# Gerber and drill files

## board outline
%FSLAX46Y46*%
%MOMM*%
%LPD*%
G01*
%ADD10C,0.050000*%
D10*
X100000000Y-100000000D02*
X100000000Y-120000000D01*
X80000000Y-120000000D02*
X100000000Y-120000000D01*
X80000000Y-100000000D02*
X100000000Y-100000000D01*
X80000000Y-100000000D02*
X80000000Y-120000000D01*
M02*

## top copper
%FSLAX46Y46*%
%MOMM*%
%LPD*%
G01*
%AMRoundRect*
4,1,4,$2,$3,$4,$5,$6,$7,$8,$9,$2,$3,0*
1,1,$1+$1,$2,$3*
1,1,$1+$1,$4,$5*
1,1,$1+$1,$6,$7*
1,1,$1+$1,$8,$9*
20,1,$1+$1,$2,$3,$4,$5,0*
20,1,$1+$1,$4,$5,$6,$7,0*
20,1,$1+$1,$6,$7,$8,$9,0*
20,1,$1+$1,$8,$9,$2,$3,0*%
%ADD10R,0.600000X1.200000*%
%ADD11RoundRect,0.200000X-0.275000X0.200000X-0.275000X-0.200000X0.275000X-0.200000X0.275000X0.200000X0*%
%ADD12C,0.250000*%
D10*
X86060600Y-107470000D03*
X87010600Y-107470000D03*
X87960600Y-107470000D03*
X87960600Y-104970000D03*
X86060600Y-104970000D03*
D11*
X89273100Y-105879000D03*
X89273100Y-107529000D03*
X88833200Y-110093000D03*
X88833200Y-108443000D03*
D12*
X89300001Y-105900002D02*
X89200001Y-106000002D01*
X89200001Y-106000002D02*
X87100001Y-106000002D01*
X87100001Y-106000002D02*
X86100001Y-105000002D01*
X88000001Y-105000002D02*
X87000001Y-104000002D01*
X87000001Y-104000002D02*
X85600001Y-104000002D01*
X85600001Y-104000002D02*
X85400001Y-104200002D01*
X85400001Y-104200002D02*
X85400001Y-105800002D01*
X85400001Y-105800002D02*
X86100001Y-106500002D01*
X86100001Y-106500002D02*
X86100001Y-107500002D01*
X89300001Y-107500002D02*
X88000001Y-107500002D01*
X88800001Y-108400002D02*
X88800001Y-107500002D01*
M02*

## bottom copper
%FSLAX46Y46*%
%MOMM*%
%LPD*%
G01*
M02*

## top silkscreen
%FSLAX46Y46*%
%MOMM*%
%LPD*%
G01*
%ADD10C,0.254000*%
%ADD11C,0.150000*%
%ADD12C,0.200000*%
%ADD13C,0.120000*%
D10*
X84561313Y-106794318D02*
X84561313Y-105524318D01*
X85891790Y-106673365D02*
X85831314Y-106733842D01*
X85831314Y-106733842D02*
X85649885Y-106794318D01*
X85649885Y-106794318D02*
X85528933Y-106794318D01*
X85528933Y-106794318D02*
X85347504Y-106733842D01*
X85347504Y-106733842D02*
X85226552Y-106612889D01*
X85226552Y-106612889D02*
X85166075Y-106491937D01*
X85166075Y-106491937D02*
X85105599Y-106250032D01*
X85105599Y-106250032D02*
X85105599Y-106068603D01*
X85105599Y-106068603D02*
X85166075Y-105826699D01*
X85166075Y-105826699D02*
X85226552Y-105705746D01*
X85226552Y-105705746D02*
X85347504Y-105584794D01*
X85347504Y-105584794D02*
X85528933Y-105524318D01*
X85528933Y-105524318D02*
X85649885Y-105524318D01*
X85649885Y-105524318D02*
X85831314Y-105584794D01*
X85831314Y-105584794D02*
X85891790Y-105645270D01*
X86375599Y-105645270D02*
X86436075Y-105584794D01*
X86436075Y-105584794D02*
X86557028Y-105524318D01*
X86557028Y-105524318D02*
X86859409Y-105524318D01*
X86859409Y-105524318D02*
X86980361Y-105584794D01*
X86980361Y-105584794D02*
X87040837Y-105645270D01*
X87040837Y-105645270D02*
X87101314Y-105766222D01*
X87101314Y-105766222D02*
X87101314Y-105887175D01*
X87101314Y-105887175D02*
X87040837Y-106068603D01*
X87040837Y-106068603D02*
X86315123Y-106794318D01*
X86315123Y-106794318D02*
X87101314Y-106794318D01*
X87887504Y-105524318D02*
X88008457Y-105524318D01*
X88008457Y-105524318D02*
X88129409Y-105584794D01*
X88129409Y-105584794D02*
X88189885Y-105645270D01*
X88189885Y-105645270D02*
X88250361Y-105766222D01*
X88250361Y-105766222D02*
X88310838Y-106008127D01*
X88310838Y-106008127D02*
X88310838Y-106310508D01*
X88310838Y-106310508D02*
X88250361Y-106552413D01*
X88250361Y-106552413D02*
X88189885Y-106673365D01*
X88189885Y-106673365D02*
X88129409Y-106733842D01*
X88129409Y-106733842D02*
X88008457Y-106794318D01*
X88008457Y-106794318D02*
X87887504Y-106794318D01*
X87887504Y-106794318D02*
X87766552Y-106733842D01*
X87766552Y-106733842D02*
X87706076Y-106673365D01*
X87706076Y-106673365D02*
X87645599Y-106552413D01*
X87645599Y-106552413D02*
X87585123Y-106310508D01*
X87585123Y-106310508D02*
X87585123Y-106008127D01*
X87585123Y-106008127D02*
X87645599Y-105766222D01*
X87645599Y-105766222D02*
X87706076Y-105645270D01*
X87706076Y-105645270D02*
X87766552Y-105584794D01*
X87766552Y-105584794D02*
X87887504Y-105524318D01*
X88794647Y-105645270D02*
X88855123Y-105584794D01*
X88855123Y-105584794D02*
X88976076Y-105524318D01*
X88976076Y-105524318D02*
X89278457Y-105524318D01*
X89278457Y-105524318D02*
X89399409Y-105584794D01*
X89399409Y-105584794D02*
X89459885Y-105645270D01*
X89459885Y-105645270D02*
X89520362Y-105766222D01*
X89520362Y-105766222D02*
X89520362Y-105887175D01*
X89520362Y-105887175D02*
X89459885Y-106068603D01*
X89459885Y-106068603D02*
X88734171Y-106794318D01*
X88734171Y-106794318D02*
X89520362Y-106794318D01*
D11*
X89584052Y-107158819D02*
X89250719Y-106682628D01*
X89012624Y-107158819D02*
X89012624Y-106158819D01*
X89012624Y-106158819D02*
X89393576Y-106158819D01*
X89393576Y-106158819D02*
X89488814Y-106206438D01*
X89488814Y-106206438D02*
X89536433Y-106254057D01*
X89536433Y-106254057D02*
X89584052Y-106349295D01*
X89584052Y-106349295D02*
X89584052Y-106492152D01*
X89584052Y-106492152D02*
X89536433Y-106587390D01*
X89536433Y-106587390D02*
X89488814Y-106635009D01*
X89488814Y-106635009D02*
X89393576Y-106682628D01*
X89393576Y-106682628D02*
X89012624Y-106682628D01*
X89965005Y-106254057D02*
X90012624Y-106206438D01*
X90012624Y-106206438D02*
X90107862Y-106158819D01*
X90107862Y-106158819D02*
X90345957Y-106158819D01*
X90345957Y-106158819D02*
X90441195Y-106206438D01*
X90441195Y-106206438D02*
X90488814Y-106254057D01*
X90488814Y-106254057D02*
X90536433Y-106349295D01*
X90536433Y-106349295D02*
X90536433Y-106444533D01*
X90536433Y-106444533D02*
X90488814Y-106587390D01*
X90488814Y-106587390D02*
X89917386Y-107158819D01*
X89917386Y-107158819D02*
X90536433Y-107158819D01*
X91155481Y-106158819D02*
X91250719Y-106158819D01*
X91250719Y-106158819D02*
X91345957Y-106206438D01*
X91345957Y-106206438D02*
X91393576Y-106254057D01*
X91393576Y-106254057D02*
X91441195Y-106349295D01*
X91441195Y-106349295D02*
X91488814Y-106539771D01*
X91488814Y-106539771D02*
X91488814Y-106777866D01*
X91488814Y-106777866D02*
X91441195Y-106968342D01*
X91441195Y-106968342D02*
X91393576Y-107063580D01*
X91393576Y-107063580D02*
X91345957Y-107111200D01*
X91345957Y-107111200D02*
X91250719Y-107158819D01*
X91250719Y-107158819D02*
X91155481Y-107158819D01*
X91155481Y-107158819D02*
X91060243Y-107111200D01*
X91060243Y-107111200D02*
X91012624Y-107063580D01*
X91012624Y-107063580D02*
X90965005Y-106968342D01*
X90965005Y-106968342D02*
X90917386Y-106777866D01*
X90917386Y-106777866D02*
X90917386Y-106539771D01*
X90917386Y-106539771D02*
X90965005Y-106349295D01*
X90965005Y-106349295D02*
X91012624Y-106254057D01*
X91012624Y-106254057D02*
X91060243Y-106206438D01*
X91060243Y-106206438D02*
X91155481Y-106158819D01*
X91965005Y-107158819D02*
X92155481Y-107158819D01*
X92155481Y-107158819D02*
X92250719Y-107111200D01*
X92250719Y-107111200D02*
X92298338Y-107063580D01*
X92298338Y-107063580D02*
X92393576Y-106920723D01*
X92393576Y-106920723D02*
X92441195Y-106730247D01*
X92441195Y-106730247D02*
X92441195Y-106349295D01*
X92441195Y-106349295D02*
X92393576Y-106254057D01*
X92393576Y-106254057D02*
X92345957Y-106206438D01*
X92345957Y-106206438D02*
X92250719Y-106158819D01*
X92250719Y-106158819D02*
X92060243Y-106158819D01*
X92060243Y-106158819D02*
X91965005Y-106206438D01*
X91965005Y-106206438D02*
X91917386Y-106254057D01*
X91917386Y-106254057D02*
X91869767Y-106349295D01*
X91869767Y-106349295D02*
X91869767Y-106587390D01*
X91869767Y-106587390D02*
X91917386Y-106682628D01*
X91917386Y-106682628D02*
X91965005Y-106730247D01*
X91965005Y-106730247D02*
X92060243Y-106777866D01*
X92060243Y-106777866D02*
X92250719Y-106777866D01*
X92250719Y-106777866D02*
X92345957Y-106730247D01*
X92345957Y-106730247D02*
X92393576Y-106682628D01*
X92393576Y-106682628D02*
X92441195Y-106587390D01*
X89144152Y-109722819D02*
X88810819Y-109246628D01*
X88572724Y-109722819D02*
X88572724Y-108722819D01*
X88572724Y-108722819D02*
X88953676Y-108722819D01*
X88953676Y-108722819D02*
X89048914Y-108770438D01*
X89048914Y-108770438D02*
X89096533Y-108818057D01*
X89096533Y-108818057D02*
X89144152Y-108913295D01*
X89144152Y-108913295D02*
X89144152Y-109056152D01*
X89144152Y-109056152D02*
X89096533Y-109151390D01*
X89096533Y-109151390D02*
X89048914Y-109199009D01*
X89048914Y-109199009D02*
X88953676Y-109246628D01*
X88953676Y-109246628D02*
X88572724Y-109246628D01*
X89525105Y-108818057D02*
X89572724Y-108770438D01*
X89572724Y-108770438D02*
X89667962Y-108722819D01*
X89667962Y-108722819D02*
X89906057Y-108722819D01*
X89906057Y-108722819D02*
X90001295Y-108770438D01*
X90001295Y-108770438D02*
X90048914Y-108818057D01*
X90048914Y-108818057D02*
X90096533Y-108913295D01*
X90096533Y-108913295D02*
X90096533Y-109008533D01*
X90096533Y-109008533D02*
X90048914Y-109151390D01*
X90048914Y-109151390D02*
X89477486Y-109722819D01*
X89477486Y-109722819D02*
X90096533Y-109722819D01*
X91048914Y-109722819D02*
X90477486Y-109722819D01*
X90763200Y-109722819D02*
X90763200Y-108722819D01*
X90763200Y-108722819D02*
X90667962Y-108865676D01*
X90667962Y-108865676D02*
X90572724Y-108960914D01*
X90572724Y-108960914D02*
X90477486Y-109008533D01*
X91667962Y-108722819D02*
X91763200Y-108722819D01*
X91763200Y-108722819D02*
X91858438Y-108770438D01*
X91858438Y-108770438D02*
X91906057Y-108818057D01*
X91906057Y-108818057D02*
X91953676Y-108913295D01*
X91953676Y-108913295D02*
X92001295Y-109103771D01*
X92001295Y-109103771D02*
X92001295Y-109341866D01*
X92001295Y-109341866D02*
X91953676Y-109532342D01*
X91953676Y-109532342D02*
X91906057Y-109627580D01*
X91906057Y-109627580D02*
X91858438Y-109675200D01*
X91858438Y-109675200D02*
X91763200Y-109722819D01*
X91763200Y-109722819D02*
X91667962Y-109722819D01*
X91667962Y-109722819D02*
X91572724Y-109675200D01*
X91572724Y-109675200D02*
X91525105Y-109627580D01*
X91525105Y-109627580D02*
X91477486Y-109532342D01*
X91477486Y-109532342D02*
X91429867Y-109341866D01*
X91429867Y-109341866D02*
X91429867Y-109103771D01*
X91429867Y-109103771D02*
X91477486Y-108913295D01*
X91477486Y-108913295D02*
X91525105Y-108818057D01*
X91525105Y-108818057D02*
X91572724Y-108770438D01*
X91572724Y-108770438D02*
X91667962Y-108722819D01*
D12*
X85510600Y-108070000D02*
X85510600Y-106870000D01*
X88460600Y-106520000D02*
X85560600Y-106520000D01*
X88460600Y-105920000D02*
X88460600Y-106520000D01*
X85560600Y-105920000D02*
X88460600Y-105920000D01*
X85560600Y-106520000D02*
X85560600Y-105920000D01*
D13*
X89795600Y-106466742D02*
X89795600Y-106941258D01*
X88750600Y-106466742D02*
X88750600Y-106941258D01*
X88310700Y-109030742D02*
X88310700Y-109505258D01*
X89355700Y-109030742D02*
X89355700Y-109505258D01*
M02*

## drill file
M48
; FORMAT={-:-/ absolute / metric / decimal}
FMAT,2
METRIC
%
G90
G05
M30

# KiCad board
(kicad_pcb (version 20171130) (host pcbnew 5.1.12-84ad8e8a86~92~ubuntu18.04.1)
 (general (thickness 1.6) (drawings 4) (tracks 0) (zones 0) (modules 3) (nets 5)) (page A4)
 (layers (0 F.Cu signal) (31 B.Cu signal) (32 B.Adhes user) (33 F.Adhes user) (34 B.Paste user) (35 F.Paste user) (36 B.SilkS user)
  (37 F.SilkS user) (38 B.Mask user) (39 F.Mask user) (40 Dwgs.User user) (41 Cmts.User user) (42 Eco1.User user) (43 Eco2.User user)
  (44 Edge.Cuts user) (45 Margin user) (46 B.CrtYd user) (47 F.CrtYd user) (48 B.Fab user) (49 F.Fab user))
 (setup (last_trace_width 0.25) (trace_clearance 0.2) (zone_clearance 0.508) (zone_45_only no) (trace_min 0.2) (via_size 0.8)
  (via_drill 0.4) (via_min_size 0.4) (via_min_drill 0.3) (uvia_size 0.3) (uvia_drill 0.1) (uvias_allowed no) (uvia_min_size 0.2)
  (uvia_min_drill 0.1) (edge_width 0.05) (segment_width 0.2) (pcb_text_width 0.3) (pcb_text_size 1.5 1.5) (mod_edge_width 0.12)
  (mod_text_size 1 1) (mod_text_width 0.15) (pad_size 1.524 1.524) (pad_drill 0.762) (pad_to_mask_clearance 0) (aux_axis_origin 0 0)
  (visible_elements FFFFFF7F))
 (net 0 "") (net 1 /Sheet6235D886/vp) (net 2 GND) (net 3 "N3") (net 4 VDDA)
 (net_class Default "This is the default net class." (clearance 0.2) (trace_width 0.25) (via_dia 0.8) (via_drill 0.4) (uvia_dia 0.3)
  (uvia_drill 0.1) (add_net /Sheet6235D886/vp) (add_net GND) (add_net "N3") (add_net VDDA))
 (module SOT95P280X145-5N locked (layer F.Cu) (at 87.010600 106.220000 90.000000)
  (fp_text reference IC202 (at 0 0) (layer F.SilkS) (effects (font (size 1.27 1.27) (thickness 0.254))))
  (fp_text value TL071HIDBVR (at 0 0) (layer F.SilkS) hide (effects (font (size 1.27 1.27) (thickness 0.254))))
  (fp_line (start -1.85 -1.5) (end -0.65 -1.5) (layer F.SilkS) (width 0.2))
  (fp_line (start -0.3 1.45) (end -0.3 -1.45) (layer F.SilkS) (width 0.2))
  (fp_line (start 0.3 1.45) (end -0.3 1.45) (layer F.SilkS) (width 0.2))
  (fp_line (start 0.3 -1.45) (end 0.3 1.45) (layer F.SilkS) (width 0.2))
  (fp_line (start -0.3 -1.45) (end 0.3 -1.45) (layer F.SilkS) (width 0.2))
  (pad 1 smd rect (at -1.25 -0.95 180.000000) (size 0.6 1.2) (layers F.Cu F.Mask F.Paste) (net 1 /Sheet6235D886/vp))
  (pad 2 smd rect (at -1.25 0 180.000000) (size 0.6 1.2) (layers F.Cu F.Mask F.Paste) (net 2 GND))
  (pad 3 smd rect (at -1.25 0.95 180.000000) (size 0.6 1.2) (layers F.Cu F.Mask F.Paste) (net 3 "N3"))
  (pad 4 smd rect (at 1.25 0.95 180.000000) (size 0.6 1.2) (layers F.Cu F.Mask F.Paste) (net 1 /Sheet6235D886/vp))
  (pad 5 smd rect (at 1.25 -0.95 180.000000) (size 0.6 1.2) (layers F.Cu F.Mask F.Paste) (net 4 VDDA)))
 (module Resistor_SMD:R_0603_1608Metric (layer F.Cu) (at 89.273100 106.704000 270.000000)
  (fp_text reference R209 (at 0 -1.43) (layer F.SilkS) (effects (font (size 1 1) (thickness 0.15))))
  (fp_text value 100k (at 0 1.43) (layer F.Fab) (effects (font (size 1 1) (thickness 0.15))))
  (fp_line (start -0.237258 -0.5225) (end 0.237258 -0.5225) (layer F.SilkS) (width 0.12))
  (fp_line (start -0.237258 0.5225) (end 0.237258 0.5225) (layer F.SilkS) (width 0.12))
  (pad 1 smd roundrect (at -0.825 0 270.000000) (size 0.8 0.95) (layers F.Cu F.Mask F.Paste) (roundrect_rratio 0.25) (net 4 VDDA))
  (pad 2 smd roundrect (at 0.825 0 270.000000) (size 0.8 0.95) (layers F.Cu F.Mask F.Paste) (roundrect_rratio 0.25) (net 3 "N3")))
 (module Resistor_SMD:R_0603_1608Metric (layer F.Cu) (at 88.833200 109.268000 270.000000)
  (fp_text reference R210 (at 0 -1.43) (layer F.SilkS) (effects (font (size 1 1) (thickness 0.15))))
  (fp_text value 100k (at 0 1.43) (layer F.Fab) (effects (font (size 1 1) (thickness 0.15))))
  (fp_line (start -0.237258 0.5225) (end 0.237258 0.5225) (layer F.SilkS) (width 0.12))
  (fp_line (start -0.237258 -0.5225) (end 0.237258 -0.5225) (layer F.SilkS) (width 0.12))
  (pad 2 smd roundrect (at 0.825 0 270.000000) (size 0.8 0.95) (layers F.Cu F.Mask F.Paste) (roundrect_rratio 0.25) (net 2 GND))
  (pad 1 smd roundrect (at -0.825 0 270.000000) (size 0.8 0.95) (layers F.Cu F.Mask F.Paste) (roundrect_rratio 0.25) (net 3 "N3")))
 (gr_line (start 100 100) (end 100 120) (layer Edge.Cuts) (width 0.05))
 (gr_line (start 80 120) (end 100 120) (layer Edge.Cuts) (width 0.05))
 (gr_line (start 80 100) (end 100 100) (layer Edge.Cuts) (width 0.05))
 (gr_line (start 80 100) (end 80 120) (layer Edge.Cuts) (width 0.05))
 (segment (start 89.300001 105.900002) (end 89.200001 106.000002) (width 0.250000) (layer F.Cu) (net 4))
 (segment (start 89.200001 106.000002) (end 87.100001 106.000002) (width 0.250000) (layer F.Cu) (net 4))
 (segment (start 87.100001 106.000002) (end 86.100001 105.000002) (width 0.250000) (layer F.Cu) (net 4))
 (segment (start 88.000001 105.000002) (end 87.000001 104.000002) (width 0.250000) (layer F.Cu) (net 1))
 (segment (start 87.000001 104.000002) (end 85.600001 104.000002) (width 0.250000) (layer F.Cu) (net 1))
 (segment (start 85.600001 104.000002) (end 85.400001 104.200002) (width 0.250000) (layer F.Cu) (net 1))
 (segment (start 85.400001 104.200002) (end 85.400001 105.800002) (width 0.250000) (layer F.Cu) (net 1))
 (segment (start 85.400001 105.800002) (end 86.100001 106.500002) (width 0.250000) (layer F.Cu) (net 1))
 (segment (start 86.100001 106.500002) (end 86.100001 107.500002) (width 0.250000) (layer F.Cu) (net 1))
 (segment (start 89.300001 107.500002) (end 88.000001 107.500002) (width 0.250000) (layer F.Cu) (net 3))
 (segment (start 88.800001 108.400002) (end 88.800001 107.500002) (width 0.250000) (layer F.Cu) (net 3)))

